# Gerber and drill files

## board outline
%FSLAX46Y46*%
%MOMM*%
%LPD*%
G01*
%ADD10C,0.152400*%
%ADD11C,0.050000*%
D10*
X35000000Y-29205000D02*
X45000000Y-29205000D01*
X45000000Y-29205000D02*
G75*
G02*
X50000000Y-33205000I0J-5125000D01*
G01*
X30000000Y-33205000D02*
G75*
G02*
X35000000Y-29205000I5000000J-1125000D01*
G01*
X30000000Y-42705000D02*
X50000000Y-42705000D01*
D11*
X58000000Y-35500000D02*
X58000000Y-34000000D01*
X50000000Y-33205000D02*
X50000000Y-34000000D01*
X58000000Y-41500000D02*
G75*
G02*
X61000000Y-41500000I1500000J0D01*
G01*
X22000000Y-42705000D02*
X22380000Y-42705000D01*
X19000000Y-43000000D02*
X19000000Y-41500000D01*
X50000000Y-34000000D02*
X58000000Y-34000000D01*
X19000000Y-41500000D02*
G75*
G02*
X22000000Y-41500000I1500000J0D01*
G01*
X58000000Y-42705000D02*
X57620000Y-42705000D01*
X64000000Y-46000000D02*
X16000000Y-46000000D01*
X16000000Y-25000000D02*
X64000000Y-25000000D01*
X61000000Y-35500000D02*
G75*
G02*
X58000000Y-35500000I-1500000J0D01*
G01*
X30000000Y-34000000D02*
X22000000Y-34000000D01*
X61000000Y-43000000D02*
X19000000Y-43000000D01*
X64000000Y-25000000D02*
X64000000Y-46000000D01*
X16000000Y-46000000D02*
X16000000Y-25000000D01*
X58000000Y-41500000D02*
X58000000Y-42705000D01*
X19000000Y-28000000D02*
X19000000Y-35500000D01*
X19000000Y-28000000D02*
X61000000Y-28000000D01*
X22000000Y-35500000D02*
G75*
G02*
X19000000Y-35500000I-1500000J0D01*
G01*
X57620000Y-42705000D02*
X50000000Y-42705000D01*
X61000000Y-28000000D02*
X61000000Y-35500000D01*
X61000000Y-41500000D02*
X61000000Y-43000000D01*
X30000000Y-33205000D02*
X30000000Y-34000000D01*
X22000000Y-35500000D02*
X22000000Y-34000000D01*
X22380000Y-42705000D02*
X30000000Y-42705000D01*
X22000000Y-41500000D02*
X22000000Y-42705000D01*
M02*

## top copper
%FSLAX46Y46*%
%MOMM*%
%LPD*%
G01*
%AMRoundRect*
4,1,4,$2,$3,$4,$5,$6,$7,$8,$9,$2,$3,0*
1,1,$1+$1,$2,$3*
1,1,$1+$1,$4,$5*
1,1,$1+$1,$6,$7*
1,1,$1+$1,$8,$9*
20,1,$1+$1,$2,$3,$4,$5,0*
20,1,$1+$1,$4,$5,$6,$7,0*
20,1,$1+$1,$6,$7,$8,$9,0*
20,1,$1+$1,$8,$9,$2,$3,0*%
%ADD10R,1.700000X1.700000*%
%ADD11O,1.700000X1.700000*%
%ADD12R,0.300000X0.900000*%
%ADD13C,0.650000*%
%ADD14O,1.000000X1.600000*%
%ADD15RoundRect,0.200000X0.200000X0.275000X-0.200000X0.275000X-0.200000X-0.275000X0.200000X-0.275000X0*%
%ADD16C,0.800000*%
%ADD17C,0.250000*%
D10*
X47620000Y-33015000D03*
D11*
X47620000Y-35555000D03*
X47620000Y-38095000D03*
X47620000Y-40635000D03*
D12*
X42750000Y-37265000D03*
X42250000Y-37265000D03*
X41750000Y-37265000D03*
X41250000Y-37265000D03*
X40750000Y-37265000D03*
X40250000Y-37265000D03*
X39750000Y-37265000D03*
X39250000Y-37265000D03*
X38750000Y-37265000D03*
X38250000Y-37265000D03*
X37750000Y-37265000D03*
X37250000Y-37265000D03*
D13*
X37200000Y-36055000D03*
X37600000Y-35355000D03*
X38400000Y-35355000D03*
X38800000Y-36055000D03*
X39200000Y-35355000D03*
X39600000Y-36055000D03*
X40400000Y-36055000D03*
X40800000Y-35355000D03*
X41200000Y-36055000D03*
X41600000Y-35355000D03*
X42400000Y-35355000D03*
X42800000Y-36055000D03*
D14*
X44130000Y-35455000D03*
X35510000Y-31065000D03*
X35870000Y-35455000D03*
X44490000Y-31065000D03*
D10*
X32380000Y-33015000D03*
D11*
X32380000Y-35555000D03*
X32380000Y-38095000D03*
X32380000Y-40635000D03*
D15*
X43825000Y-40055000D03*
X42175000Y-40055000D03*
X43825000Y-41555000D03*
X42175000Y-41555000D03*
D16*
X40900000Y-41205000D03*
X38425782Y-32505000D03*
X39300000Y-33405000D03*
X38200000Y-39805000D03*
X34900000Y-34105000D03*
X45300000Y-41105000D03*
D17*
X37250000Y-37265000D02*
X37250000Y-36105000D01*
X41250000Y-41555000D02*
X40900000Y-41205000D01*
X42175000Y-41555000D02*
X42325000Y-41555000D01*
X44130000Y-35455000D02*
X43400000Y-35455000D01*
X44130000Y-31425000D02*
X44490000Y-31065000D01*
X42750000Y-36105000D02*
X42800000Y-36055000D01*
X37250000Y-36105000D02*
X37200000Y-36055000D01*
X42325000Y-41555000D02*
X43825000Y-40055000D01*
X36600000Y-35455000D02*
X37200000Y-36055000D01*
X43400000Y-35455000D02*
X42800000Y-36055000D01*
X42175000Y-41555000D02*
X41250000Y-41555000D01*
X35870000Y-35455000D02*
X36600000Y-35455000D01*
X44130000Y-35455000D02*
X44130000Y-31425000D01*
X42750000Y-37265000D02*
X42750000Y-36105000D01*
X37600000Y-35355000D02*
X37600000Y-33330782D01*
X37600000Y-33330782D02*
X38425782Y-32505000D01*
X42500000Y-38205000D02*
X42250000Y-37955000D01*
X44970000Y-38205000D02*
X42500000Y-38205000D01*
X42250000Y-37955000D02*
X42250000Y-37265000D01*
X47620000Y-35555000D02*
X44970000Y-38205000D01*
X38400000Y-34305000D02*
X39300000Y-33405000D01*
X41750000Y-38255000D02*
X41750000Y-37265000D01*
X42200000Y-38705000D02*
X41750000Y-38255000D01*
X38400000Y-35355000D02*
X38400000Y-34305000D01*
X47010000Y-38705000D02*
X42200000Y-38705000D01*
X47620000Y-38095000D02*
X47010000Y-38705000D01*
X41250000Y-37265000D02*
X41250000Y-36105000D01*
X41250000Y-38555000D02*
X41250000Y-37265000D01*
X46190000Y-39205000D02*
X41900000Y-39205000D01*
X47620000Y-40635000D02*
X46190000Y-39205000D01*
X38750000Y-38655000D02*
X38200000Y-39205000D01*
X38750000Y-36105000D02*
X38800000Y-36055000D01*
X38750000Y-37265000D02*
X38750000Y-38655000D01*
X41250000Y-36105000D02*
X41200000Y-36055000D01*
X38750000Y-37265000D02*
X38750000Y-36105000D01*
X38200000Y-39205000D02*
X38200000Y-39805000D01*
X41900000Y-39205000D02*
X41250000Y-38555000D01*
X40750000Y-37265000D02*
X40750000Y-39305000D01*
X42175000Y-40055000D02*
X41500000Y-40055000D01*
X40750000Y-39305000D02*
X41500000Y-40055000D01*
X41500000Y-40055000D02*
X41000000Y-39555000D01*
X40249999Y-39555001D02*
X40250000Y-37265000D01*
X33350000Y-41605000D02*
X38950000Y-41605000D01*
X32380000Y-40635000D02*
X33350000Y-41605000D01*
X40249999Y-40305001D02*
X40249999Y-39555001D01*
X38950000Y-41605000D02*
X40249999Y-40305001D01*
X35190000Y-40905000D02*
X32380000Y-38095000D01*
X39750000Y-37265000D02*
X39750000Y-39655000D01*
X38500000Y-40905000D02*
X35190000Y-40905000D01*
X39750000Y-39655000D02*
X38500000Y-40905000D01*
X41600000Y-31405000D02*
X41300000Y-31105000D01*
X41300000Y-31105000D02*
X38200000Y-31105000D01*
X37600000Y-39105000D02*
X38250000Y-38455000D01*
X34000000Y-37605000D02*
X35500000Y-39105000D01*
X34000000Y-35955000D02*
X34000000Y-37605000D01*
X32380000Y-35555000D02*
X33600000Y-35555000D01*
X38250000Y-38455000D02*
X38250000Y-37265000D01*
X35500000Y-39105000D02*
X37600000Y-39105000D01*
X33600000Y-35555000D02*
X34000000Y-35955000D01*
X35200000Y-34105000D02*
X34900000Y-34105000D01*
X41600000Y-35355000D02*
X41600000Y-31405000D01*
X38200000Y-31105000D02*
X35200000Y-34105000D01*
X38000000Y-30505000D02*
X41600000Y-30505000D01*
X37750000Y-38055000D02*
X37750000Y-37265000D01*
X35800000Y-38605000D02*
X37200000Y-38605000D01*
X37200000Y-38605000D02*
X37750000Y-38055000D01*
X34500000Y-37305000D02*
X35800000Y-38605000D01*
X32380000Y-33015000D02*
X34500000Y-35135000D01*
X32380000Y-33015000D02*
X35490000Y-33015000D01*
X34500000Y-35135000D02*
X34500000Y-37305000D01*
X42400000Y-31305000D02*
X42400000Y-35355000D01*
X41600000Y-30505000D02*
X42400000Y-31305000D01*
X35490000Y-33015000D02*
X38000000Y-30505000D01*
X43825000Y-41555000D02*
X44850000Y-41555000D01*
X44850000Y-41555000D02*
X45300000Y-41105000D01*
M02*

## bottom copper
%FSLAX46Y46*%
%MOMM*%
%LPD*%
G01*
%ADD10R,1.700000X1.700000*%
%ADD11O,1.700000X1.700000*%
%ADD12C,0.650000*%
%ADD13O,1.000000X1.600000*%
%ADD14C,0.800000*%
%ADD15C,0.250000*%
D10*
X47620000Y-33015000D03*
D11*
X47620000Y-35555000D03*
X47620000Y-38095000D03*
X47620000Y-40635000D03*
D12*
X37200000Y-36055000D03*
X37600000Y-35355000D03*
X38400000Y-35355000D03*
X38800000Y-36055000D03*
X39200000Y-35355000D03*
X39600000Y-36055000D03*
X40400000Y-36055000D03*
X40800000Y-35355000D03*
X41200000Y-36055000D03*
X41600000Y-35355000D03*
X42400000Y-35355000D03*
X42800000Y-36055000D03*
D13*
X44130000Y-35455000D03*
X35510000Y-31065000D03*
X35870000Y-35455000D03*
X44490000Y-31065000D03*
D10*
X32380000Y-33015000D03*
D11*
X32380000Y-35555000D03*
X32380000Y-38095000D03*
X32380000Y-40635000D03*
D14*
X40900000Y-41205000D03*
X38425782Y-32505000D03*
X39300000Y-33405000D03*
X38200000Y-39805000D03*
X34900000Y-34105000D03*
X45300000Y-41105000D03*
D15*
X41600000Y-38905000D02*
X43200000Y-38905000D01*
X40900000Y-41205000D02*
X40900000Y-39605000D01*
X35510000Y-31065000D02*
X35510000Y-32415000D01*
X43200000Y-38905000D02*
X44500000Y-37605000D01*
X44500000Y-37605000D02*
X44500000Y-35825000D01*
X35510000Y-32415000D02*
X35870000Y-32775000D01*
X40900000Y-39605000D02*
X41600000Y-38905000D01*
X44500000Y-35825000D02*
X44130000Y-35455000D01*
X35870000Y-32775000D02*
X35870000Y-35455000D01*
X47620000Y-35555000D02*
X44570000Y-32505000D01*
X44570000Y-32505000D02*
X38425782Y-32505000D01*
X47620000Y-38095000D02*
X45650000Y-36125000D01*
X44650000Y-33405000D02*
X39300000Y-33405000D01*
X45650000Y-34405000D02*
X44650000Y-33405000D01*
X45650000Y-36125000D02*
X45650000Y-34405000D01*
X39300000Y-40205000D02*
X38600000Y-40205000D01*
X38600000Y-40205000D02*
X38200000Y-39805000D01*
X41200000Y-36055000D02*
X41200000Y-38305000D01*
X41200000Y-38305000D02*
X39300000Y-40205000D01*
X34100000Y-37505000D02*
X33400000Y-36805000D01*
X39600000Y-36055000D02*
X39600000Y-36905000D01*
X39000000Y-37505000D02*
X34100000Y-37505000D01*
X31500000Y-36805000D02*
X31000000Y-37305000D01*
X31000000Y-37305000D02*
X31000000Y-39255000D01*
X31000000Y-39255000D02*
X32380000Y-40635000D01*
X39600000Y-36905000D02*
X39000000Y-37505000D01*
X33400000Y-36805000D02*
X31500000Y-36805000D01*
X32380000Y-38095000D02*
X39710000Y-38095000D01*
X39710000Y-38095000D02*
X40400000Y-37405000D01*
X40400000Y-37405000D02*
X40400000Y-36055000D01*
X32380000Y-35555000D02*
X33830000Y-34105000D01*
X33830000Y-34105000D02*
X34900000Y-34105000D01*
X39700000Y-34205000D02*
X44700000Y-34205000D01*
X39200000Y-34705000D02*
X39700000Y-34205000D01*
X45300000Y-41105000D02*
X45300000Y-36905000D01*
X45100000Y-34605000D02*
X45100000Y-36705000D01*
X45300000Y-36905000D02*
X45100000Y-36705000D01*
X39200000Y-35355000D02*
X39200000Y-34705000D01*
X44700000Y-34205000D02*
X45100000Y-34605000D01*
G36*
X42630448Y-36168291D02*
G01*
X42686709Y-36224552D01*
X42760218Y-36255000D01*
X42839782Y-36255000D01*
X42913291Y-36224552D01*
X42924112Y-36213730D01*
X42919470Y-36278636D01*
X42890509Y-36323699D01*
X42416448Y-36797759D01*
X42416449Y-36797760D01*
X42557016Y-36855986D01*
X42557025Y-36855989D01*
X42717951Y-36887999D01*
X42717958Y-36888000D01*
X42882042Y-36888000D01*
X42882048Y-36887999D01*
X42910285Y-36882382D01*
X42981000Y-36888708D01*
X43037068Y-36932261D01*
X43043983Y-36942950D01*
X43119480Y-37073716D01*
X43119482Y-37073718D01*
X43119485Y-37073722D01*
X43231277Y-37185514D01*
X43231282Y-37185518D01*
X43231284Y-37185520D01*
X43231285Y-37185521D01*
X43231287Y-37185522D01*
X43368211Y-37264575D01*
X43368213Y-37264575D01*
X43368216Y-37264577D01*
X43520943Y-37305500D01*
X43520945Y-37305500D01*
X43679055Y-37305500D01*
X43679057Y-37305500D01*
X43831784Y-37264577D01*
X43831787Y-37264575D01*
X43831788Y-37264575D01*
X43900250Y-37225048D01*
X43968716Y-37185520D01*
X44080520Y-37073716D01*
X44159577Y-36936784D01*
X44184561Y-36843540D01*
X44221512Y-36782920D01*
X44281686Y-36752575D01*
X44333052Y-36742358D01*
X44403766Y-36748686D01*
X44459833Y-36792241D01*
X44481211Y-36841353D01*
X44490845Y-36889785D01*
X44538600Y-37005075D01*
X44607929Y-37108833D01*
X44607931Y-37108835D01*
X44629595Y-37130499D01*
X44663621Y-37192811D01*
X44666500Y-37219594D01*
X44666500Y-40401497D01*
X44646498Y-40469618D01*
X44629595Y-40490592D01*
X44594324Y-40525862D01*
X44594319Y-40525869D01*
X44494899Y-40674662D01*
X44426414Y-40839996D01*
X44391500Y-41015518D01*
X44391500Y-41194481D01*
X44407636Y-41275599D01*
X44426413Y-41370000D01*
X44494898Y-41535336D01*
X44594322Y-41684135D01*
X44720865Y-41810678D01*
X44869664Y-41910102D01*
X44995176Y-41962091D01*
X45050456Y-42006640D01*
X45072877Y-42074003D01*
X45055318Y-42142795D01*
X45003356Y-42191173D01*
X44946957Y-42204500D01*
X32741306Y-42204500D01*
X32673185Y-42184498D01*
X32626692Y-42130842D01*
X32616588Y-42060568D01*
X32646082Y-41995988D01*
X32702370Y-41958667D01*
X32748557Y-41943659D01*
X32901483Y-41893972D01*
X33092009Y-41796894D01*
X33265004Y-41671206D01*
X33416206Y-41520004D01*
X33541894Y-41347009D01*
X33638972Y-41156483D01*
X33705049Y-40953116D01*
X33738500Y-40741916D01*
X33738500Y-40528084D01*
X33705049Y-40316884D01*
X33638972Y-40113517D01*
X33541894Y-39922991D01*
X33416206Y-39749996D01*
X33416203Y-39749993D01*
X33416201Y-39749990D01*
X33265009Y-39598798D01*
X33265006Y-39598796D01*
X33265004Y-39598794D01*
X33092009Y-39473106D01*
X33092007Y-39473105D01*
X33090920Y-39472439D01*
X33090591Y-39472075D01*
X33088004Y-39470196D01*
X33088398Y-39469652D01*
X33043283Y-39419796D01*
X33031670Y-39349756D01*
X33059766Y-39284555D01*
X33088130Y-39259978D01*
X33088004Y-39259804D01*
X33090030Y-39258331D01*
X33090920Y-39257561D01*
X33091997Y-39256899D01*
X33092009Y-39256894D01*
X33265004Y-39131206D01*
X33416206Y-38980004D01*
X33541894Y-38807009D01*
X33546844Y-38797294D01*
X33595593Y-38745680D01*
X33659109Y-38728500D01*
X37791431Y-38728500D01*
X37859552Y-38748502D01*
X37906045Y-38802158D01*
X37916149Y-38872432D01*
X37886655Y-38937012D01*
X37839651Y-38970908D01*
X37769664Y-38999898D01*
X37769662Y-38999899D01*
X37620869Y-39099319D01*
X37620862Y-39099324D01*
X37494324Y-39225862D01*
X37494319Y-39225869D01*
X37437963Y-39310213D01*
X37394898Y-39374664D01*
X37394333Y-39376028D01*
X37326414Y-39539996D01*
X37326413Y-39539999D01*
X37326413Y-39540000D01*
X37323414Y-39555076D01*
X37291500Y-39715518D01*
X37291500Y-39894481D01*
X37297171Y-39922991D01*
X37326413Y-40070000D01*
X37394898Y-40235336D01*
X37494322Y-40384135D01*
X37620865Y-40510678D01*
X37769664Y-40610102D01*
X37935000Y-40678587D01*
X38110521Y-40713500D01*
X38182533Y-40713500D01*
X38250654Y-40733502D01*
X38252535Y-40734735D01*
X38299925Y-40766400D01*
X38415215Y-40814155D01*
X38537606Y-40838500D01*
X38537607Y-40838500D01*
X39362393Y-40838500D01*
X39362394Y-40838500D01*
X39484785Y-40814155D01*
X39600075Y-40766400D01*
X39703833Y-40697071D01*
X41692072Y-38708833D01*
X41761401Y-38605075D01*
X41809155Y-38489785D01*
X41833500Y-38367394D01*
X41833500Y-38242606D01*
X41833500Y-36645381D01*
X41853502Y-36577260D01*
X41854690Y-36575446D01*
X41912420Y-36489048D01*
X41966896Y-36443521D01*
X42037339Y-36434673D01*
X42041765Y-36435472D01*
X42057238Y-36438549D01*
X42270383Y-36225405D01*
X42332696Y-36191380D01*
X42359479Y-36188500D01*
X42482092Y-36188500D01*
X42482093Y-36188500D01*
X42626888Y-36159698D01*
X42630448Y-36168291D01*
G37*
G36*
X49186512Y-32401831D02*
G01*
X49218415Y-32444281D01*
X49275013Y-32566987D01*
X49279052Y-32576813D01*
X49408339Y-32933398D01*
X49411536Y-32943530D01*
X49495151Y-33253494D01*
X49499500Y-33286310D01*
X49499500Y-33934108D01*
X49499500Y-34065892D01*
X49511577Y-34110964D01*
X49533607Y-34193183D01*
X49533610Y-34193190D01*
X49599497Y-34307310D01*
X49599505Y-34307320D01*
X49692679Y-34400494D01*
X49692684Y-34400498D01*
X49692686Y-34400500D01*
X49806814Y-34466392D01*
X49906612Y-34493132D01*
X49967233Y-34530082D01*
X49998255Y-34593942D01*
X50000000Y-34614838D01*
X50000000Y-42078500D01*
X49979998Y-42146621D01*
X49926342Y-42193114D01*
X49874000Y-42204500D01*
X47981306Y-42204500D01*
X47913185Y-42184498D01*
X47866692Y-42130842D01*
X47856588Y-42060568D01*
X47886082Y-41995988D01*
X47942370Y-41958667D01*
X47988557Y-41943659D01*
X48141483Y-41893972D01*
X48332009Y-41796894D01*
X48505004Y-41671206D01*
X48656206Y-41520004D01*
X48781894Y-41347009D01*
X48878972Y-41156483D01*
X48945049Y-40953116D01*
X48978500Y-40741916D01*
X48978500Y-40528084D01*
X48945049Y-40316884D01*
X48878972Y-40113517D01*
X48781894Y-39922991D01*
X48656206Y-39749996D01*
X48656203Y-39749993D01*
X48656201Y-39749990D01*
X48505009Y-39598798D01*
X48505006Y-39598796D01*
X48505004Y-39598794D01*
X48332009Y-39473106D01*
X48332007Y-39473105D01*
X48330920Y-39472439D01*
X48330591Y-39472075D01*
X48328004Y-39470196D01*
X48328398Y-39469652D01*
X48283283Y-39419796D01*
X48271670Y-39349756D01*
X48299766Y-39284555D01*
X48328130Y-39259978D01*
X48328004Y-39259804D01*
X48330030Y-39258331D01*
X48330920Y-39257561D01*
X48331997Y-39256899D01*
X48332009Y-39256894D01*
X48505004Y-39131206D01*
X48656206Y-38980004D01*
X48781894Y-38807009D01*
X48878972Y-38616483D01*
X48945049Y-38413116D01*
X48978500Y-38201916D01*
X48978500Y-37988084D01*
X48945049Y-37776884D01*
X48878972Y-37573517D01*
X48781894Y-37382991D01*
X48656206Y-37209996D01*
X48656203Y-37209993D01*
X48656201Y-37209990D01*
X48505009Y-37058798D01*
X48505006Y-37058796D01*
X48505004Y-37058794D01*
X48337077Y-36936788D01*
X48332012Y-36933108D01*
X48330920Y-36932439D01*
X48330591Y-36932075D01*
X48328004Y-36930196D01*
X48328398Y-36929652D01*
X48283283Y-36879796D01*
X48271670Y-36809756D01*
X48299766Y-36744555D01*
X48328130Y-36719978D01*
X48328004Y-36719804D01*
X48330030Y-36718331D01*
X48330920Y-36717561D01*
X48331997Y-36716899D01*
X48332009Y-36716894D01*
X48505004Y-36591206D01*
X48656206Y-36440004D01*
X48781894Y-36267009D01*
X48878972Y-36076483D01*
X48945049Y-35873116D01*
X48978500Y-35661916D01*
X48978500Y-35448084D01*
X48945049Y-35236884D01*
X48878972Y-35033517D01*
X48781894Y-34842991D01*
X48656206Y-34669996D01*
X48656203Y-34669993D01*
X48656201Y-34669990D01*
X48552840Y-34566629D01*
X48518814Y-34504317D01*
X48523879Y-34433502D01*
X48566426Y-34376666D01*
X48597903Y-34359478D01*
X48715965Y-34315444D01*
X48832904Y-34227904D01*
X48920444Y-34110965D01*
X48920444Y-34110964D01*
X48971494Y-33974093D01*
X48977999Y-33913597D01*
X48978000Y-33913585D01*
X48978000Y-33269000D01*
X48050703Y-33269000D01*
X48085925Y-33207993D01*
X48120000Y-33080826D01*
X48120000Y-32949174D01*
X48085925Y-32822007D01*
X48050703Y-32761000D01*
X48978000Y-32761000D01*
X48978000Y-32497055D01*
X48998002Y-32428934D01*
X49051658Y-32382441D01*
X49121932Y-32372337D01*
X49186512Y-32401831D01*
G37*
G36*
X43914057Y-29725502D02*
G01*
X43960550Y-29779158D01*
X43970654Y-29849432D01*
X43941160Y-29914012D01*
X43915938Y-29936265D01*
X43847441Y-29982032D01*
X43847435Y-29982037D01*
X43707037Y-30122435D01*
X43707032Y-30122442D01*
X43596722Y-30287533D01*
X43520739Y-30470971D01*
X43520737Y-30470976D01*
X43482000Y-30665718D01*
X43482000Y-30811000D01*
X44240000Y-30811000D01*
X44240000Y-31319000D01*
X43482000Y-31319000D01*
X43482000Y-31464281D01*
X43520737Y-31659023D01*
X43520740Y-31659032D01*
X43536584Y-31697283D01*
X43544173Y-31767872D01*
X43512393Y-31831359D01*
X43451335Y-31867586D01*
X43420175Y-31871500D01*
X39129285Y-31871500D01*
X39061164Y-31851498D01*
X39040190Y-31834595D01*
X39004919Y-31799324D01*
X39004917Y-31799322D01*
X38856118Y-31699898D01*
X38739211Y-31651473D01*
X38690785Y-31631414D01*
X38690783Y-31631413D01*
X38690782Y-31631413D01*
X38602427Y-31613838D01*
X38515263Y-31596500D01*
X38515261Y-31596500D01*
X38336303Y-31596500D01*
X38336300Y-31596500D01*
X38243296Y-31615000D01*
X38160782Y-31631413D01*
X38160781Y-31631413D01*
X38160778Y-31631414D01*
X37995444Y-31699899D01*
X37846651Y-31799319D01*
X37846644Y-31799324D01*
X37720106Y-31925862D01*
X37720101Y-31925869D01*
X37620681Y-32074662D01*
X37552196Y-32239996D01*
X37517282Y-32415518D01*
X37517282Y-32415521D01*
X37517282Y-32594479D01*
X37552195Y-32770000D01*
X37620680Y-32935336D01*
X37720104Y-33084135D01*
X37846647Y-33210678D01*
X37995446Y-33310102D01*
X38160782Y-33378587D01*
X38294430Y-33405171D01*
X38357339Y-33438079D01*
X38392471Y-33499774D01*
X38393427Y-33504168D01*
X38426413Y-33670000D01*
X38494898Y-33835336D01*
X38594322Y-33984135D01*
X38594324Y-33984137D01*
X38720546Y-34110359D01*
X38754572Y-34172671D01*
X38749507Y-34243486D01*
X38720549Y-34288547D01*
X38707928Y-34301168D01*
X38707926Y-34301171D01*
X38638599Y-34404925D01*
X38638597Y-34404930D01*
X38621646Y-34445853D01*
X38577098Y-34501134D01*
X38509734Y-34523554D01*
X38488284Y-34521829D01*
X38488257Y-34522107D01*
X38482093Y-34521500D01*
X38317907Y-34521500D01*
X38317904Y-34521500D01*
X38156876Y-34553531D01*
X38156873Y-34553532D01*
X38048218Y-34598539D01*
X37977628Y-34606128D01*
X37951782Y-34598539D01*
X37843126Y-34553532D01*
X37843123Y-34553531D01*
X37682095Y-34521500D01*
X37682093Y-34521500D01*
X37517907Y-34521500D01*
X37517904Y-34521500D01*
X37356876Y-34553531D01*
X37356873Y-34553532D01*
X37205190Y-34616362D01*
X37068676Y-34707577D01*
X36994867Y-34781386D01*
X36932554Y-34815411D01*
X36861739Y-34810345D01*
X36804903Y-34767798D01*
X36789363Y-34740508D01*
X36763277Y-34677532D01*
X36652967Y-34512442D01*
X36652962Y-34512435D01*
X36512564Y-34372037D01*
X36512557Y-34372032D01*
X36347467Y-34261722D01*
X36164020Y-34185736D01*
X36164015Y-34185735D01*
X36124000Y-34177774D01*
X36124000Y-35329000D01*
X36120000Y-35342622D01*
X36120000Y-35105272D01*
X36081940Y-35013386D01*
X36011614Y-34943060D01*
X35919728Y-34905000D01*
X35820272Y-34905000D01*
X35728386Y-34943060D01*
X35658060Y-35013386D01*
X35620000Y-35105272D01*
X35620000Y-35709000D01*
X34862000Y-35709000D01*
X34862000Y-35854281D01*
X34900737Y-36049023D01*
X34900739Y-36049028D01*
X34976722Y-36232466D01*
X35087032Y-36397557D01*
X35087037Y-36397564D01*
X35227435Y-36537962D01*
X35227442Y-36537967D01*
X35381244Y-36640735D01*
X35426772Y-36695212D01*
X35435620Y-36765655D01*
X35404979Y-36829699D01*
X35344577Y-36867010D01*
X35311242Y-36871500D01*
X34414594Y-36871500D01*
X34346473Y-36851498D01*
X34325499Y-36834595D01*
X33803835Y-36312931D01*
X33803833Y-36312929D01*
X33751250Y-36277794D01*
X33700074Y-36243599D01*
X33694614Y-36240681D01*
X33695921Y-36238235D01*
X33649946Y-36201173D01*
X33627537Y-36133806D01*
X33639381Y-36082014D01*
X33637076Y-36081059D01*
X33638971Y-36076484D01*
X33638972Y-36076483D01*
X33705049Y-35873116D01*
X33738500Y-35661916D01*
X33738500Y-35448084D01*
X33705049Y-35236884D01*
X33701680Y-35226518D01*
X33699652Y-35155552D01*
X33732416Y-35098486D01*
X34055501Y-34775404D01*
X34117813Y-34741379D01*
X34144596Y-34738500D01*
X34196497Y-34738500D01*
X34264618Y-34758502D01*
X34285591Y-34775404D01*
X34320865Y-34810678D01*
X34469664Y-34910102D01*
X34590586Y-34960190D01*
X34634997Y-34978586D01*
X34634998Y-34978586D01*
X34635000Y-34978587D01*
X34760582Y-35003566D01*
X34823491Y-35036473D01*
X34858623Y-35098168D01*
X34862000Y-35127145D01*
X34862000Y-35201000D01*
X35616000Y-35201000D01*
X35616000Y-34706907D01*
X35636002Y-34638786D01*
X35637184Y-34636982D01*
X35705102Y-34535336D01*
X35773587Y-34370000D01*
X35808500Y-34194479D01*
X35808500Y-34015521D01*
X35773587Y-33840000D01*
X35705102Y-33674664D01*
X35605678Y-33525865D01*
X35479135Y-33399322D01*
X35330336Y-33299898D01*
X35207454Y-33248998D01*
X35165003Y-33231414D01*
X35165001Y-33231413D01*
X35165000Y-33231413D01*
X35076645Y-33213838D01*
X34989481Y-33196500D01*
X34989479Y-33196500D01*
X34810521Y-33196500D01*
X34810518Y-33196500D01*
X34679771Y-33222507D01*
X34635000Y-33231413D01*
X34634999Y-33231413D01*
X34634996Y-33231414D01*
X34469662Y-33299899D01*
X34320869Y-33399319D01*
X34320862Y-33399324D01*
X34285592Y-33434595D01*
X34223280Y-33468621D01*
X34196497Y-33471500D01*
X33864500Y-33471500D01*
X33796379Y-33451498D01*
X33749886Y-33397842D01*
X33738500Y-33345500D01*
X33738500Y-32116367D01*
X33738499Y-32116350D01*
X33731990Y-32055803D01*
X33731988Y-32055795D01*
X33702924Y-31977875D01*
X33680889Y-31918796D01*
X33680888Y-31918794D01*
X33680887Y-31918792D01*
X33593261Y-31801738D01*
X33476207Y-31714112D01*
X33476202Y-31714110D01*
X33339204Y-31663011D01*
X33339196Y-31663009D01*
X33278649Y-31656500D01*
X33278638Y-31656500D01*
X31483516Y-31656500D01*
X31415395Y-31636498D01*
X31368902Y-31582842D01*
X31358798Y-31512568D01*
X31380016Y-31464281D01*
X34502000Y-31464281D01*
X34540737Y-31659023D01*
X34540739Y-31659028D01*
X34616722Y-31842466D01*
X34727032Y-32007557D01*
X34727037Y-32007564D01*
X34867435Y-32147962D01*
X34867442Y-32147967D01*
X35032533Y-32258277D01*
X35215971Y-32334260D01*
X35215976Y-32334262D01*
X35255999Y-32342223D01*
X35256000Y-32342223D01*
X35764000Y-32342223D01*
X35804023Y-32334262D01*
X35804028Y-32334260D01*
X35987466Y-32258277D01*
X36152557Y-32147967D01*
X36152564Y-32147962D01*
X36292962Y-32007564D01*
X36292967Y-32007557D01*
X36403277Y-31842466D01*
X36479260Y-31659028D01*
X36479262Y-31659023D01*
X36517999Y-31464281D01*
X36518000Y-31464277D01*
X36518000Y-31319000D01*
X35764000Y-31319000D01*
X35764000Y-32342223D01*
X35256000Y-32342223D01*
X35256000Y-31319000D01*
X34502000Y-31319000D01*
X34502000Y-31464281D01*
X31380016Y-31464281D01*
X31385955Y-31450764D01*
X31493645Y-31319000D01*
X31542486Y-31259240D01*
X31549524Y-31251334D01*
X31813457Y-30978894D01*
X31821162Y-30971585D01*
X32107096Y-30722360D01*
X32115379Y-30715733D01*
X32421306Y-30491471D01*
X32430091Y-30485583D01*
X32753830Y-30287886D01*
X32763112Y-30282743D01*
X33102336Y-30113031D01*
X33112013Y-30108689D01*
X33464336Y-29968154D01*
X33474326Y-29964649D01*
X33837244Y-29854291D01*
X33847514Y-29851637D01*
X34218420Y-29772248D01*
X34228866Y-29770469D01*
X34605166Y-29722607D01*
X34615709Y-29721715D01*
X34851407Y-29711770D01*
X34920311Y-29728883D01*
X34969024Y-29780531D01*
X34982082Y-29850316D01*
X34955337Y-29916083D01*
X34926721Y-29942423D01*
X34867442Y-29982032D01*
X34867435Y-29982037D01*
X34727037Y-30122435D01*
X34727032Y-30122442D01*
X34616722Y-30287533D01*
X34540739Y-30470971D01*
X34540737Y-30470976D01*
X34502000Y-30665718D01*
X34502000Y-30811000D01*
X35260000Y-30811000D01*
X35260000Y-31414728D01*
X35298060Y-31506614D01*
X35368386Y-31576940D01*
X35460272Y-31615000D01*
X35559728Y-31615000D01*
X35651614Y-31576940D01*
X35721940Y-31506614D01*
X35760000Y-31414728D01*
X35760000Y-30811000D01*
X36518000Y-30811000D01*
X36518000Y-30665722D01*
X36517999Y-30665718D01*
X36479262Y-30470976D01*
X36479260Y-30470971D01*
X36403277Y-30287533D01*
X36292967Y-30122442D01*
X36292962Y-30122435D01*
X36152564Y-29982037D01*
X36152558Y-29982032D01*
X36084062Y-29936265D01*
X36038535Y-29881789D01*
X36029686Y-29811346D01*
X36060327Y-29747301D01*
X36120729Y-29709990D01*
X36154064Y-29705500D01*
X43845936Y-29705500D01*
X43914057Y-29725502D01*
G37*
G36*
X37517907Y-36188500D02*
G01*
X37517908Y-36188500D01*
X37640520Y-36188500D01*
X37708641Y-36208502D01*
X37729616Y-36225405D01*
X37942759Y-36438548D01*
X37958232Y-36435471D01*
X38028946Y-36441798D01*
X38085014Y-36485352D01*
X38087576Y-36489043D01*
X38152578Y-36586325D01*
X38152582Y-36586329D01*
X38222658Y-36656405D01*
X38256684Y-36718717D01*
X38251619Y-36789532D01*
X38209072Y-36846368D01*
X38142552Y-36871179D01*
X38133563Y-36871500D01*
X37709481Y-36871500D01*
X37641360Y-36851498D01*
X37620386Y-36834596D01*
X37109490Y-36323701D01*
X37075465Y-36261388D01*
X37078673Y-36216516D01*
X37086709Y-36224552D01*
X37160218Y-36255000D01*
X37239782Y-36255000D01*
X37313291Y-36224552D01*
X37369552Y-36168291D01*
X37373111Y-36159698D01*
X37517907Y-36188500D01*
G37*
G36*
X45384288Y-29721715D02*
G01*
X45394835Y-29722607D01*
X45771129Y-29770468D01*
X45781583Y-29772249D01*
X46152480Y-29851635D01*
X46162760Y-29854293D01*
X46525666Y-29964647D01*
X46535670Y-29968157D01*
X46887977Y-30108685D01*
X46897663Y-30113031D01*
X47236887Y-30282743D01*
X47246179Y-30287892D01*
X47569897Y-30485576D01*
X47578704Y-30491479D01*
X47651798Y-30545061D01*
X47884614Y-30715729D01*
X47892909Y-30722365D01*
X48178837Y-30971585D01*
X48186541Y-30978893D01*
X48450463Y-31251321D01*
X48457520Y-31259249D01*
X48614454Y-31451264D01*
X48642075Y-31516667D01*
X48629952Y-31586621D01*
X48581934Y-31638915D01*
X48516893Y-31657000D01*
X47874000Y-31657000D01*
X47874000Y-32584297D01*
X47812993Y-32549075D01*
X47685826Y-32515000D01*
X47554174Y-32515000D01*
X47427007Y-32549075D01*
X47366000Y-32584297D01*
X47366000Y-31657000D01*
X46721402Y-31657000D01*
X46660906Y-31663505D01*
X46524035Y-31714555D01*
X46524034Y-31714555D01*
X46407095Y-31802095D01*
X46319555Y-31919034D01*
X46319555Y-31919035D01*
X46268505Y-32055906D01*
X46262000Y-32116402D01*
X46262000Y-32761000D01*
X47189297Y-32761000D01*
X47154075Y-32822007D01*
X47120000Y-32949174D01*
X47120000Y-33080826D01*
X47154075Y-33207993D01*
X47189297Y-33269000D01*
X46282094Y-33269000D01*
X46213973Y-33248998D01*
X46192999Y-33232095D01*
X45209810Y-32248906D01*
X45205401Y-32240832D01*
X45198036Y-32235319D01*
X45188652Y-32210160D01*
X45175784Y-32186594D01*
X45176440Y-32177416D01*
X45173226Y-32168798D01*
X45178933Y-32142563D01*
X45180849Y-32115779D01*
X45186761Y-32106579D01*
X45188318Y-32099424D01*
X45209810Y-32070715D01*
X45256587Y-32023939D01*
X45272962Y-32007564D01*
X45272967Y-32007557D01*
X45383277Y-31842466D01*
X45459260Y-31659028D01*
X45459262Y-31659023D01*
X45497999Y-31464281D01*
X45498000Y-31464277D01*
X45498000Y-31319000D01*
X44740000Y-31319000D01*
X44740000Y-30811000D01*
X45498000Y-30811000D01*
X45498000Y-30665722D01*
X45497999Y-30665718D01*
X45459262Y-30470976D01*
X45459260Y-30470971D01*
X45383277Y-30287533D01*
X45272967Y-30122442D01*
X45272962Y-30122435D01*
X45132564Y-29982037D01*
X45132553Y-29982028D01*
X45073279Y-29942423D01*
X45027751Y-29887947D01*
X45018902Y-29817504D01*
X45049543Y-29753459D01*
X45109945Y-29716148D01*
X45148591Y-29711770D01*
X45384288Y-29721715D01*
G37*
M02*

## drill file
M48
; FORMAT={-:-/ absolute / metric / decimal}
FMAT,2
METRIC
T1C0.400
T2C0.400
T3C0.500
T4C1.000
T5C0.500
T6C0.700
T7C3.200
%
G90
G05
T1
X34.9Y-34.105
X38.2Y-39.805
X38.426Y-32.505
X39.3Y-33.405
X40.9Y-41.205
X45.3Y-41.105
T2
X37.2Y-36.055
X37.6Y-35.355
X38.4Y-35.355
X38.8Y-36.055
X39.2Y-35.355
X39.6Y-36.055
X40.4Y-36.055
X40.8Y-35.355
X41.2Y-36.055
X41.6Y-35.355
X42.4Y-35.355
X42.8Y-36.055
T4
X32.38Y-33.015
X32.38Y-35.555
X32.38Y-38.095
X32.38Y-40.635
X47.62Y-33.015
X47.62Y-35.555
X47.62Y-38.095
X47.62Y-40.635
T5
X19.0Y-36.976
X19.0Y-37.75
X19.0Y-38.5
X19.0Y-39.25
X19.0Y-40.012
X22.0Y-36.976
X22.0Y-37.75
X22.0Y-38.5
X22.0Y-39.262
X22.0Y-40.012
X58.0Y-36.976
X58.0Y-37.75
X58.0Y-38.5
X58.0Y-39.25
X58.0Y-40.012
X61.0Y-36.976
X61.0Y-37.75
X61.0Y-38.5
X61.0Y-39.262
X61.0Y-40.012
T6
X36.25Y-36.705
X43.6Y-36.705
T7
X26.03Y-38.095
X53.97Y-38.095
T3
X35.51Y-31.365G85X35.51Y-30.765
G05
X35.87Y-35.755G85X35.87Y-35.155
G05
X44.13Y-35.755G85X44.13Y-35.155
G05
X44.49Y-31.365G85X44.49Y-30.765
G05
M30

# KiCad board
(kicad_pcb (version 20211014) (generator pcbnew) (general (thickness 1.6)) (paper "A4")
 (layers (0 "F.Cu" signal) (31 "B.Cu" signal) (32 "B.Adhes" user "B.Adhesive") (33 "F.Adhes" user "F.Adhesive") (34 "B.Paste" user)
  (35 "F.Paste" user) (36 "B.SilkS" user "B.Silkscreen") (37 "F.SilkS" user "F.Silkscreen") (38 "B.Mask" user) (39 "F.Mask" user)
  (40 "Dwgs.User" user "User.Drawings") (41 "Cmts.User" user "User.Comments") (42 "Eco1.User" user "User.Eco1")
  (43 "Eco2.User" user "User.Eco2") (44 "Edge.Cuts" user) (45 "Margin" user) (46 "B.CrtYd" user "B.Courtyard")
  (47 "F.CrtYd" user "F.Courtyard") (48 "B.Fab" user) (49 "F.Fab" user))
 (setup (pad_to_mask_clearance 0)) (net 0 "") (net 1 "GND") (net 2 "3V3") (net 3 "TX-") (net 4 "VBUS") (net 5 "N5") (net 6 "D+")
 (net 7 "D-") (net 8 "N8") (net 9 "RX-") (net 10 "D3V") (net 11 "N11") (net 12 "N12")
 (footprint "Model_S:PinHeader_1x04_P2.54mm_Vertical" (layer "F.Cu") (at 47.62 33.015)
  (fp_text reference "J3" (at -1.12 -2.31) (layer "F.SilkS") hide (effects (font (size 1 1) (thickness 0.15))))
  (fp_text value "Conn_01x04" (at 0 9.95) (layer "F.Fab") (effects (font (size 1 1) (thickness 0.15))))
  (pad "1" thru_hole rect locked (at 0 0) (size 1.7 1.7) (drill 1) (layers *.Cu *.Mask) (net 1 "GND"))
  (pad "2" thru_hole oval locked (at 0 2.54) (size 1.7 1.7) (drill 1) (layers *.Cu *.Mask) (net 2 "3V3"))
  (pad "3" thru_hole oval locked (at 0 5.08) (size 1.7 1.7) (drill 1) (layers *.Cu *.Mask) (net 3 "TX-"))
  (pad "4" thru_hole oval locked (at 0 7.62) (size 1.7 1.7) (drill 1) (layers *.Cu *.Mask) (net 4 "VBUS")))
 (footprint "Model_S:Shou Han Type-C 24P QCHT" (layer "F.Cu") (at 40 29.205 180)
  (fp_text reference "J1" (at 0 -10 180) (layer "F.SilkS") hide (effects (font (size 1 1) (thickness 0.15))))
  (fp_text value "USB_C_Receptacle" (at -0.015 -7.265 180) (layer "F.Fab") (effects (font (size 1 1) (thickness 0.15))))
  (pad "" np_thru_hole circle locked (at -3.6 -7.5 180) (size 0.7 0.7) (drill 0.7) (layers *.Cu *.Mask))
  (pad "" np_thru_hole circle locked (at 3.75 -7.5 180) (size 0.7 0.7) (drill 0.7) (layers *.Cu *.Mask))
  (pad "A1" smd rect locked (at -2.75 -8.06 180) (size 0.3 0.9) (layers "F.Cu" "F.Paste" "F.Mask") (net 1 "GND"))
  (pad "A2" smd rect locked (at -2.25 -8.06 180) (size 0.3 0.9) (layers "F.Cu" "F.Paste" "F.Mask") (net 2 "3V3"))
  (pad "A3" smd rect locked (at -1.75 -8.06 180) (size 0.3 0.9) (layers "F.Cu" "F.Paste" "F.Mask") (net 3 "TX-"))
  (pad "A4" smd rect locked (at -1.25 -8.06 180) (size 0.3 0.9) (layers "F.Cu" "F.Paste" "F.Mask") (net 4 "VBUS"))
  (pad "A5" smd rect locked (at -0.75 -8.06 180) (size 0.3 0.9) (layers "F.Cu" "F.Paste" "F.Mask") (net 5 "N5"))
  (pad "A6" smd rect locked (at -0.25 -8.06 180) (size 0.3 0.9) (layers "F.Cu" "F.Paste" "F.Mask") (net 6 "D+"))
  (pad "A7" smd rect locked (at 0.25 -8.06 180) (size 0.3 0.9) (layers "F.Cu" "F.Paste" "F.Mask") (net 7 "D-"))
  (pad "A8" smd rect locked (at 0.75 -8.06 180) (size 0.3 0.9) (layers "F.Cu" "F.Paste" "F.Mask") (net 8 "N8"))
  (pad "A9" smd rect locked (at 1.25 -8.06 180) (size 0.3 0.9) (layers "F.Cu" "F.Paste" "F.Mask") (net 4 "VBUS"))
  (pad "A10" smd rect locked (at 1.75 -8.06 180) (size 0.3 0.9) (layers "F.Cu" "F.Paste" "F.Mask") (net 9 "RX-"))
  (pad "A11" smd rect locked (at 2.25 -8.06 180) (size 0.3 0.9) (layers "F.Cu" "F.Paste" "F.Mask") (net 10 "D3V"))
  (pad "A12" smd rect locked (at 2.75 -8.06 180) (size 0.3 0.9) (layers "F.Cu" "F.Paste" "F.Mask") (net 1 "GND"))
  (pad "B1" thru_hole circle locked (at 2.8 -6.85 180) (size 0.65 0.65) (drill 0.4) (layers *.Cu *.Mask) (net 1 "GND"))
  (pad "B2" thru_hole circle locked (at 2.4 -6.15 180) (size 0.65 0.65) (drill 0.4) (layers *.Cu *.Mask) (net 2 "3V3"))
  (pad "B3" thru_hole circle locked (at 1.6 -6.15 180) (size 0.65 0.65) (drill 0.4) (layers *.Cu *.Mask) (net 3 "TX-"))
  (pad "B4" thru_hole circle locked (at 1.2 -6.85 180) (size 0.65 0.65) (drill 0.4) (layers *.Cu *.Mask) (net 4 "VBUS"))
  (pad "B5" thru_hole circle locked (at 0.8 -6.15 180) (size 0.65 0.65) (drill 0.4) (layers *.Cu *.Mask) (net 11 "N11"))
  (pad "B6" thru_hole circle locked (at 0.4 -6.85 180) (size 0.65 0.65) (drill 0.4) (layers *.Cu *.Mask) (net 6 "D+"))
  (pad "B7" thru_hole circle locked (at -0.4 -6.85 180) (size 0.65 0.65) (drill 0.4) (layers *.Cu *.Mask) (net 7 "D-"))
  (pad "B8" thru_hole circle locked (at -0.8 -6.15 180) (size 0.65 0.65) (drill 0.4) (layers *.Cu *.Mask) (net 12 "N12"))
  (pad "B9" thru_hole circle locked (at -1.2 -6.85 180) (size 0.65 0.65) (drill 0.4) (layers *.Cu *.Mask) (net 4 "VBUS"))
  (pad "B10" thru_hole circle locked (at -1.6 -6.15 180) (size 0.65 0.65) (drill 0.4) (layers *.Cu *.Mask) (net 9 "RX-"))
  (pad "B11" thru_hole circle locked (at -2.4 -6.15 180) (size 0.65 0.65) (drill 0.4) (layers *.Cu *.Mask) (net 10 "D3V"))
  (pad "B12" thru_hole circle locked (at -2.8 -6.85 180) (size 0.65 0.65) (drill 0.4) (layers *.Cu *.Mask) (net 1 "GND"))
  (pad "S1" thru_hole oval locked (at -4.13 -6.25 180) (size 1 1.6) (drill oval 0.5 1.1) (layers *.Cu *.Mask) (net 1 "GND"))
  (pad "S1" thru_hole oval locked (at 4.49 -1.86 180) (size 1 1.6) (drill oval 0.5 1.1) (layers *.Cu *.Mask) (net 1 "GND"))
  (pad "S1" thru_hole oval locked (at 4.13 -6.25 180) (size 1 1.6) (drill oval 0.5 1.1) (layers *.Cu *.Mask) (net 1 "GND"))
  (pad "S1" thru_hole oval locked (at -4.49 -1.86 180) (size 1 1.6) (drill oval 0.5 1.1) (layers *.Cu *.Mask) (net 1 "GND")))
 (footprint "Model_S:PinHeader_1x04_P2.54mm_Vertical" (layer "F.Cu") (at 32.38 33.015)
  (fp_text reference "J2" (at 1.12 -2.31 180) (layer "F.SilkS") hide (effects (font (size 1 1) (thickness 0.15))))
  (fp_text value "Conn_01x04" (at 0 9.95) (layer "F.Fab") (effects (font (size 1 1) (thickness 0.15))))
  (pad "1" thru_hole rect locked (at 0 0) (size 1.7 1.7) (drill 1) (layers *.Cu *.Mask) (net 10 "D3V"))
  (pad "2" thru_hole oval locked (at 0 2.54) (size 1.7 1.7) (drill 1) (layers *.Cu *.Mask) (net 9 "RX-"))
  (pad "3" thru_hole oval locked (at 0 5.08) (size 1.7 1.7) (drill 1) (layers *.Cu *.Mask) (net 7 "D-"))
  (pad "4" thru_hole oval locked (at 0 7.62) (size 1.7 1.7) (drill 1) (layers *.Cu *.Mask) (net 6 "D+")))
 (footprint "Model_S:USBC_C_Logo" (layer "F.Cu") (at 40 40)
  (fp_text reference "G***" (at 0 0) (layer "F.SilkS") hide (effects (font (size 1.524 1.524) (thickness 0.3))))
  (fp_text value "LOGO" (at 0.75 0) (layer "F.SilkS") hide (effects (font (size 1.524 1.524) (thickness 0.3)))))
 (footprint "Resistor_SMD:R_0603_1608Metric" (layer "F.Cu") (at 43 40.055 180)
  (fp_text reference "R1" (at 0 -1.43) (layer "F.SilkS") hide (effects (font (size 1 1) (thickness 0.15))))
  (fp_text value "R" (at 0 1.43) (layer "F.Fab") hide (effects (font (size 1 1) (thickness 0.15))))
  (pad "1" smd roundrect locked (at -0.825 0 180) (size 0.8 0.95) (layers "F.Cu" "F.Paste" "F.Mask") (roundrect_rratio 0.25) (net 1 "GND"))
  (pad "2" smd roundrect locked (at 0.825 0 180) (size 0.8 0.95) (layers "F.Cu" "F.Paste" "F.Mask") (roundrect_rratio 0.25) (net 5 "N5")))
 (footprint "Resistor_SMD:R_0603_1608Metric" (layer "F.Cu") (at 43 41.555 180)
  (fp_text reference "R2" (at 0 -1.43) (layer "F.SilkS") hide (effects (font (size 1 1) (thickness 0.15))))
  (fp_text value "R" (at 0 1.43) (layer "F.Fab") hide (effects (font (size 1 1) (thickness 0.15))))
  (pad "1" smd roundrect locked (at -0.825 0 180) (size 0.8 0.95) (layers "F.Cu" "F.Paste" "F.Mask") (roundrect_rratio 0.25) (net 11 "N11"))
  (pad "2" smd roundrect locked (at 0.825 0 180) (size 0.8 0.95) (layers "F.Cu" "F.Paste" "F.Mask") (roundrect_rratio 0.25) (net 1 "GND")))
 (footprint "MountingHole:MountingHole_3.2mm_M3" (layer "F.Cu") (at 26.03 38.095)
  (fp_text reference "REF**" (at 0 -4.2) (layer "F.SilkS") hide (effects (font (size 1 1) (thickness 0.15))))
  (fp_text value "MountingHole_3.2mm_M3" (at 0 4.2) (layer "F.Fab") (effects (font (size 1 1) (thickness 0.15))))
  (pad "" np_thru_hole circle (at 0 0) (size 3.2 3.2) (drill 3.2) (layers *.Cu *.Mask)))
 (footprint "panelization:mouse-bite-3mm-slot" (layer "F.Cu") (at 20.5 38.5 90)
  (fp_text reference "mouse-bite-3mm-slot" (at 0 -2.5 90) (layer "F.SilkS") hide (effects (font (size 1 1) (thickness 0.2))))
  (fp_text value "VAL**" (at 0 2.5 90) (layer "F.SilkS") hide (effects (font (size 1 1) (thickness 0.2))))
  (pad "" np_thru_hole circle locked (at -1.512 -1.5 90) (size 0.5 0.5) (drill 0.5) (layers *.Cu *.Mask))
  (pad "" np_thru_hole circle locked (at 0 -1.5 90) (size 0.5 0.5) (drill 0.5) (layers *.Cu *.Mask))
  (pad "" np_thru_hole circle locked (at 0.75 1.5 90) (size 0.5 0.5) (drill 0.5) (layers *.Cu *.Mask))
  (pad "" np_thru_hole circle locked (at -1.512 1.5 90) (size 0.5 0.5) (drill 0.5) (layers *.Cu *.Mask))
  (pad "" np_thru_hole circle locked (at 0 1.5 90) (size 0.5 0.5) (drill 0.5) (layers *.Cu *.Mask))
  (pad "" np_thru_hole circle locked (at -0.75 -1.5 90) (size 0.5 0.5) (drill 0.5) (layers *.Cu *.Mask))
  (pad "" np_thru_hole circle locked (at -0.762 1.5 90) (size 0.5 0.5) (drill 0.5) (layers *.Cu *.Mask))
  (pad "" np_thru_hole circle locked (at 1.524 -1.5 90) (size 0.5 0.5) (drill 0.5) (layers *.Cu *.Mask))
  (pad "" np_thru_hole circle locked (at 1.524 1.5 90) (size 0.5 0.5) (drill 0.5) (layers *.Cu *.Mask))
  (pad "" np_thru_hole circle locked (at 0.75 -1.5 90) (size 0.5 0.5) (drill 0.5) (layers *.Cu *.Mask)))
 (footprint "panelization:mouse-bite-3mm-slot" (layer "F.Cu") (at 59.5 38.5 90)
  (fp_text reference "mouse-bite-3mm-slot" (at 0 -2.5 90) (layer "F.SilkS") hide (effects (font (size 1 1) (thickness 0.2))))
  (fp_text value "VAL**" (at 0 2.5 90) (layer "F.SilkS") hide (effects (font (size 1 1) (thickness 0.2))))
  (pad "" np_thru_hole circle locked (at 0 -1.5 90) (size 0.5 0.5) (drill 0.5) (layers *.Cu *.Mask))
  (pad "" np_thru_hole circle locked (at -1.512 1.5 90) (size 0.5 0.5) (drill 0.5) (layers *.Cu *.Mask))
  (pad "" np_thru_hole circle locked (at 0.75 -1.5 90) (size 0.5 0.5) (drill 0.5) (layers *.Cu *.Mask))
  (pad "" np_thru_hole circle locked (at -1.512 -1.5 90) (size 0.5 0.5) (drill 0.5) (layers *.Cu *.Mask))
  (pad "" np_thru_hole circle locked (at 0.75 1.5 90) (size 0.5 0.5) (drill 0.5) (layers *.Cu *.Mask))
  (pad "" np_thru_hole circle locked (at -0.75 -1.5 90) (size 0.5 0.5) (drill 0.5) (layers *.Cu *.Mask))
  (pad "" np_thru_hole circle locked (at 1.524 1.5 90) (size 0.5 0.5) (drill 0.5) (layers *.Cu *.Mask))
  (pad "" np_thru_hole circle locked (at 0 1.5 90) (size 0.5 0.5) (drill 0.5) (layers *.Cu *.Mask))
  (pad "" np_thru_hole circle locked (at -0.762 1.5 90) (size 0.5 0.5) (drill 0.5) (layers *.Cu *.Mask))
  (pad "" np_thru_hole circle locked (at 1.524 -1.5 90) (size 0.5 0.5) (drill 0.5) (layers *.Cu *.Mask)))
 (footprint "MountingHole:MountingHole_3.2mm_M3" (layer "F.Cu") (at 53.97 38.095)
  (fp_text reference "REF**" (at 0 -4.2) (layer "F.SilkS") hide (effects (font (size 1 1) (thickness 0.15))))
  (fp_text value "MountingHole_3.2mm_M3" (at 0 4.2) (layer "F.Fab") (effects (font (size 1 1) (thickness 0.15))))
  (pad "" np_thru_hole circle (at 0 0) (size 3.2 3.2) (drill 3.2) (layers *.Cu *.Mask)))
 (gr_line (start 35 29.205) (end 45 29.205) (layer "Edge.Cuts") (width 0.1524))
 (gr_arc (start 45 29.205) (mid 48.201562 30.328047) (end 50 33.205) (layer "Edge.Cuts") (width 0.1524))
 (gr_arc (start 30 33.205) (mid 31.798438 30.328047) (end 35 29.205) (layer "Edge.Cuts") (width 0.1524))
 (gr_line (start 30 42.705) (end 50 42.705) (layer "Edge.Cuts") (width 0.1524))
 (gr_line (start 58 35.5) (end 58 34) (layer "Edge.Cuts") (width 0.05))
 (gr_line (start 50 33.205) (end 50 34) (layer "Edge.Cuts") (width 0.05))
 (gr_arc (start 58 41.5) (mid 59.5 40) (end 61 41.5) (layer "Edge.Cuts") (width 0.05))
 (gr_line (start 22 42.705) (end 22.38 42.705) (layer "Edge.Cuts") (width 0.05))
 (gr_line (start 19 43) (end 19 41.5) (layer "Edge.Cuts") (width 0.05))
 (gr_line (start 50 34) (end 58 34) (layer "Edge.Cuts") (width 0.05))
 (gr_arc (start 19 41.5) (mid 20.5 40) (end 22 41.5) (layer "Edge.Cuts") (width 0.05))
 (gr_line (start 58 42.705) (end 57.62 42.705) (layer "Edge.Cuts") (width 0.05))
 (gr_line (start 64 46) (end 16 46) (layer "Edge.Cuts") (width 0.05))
 (gr_line (start 16 25) (end 64 25) (layer "Edge.Cuts") (width 0.05))
 (gr_arc (start 61 35.5) (mid 59.5 37) (end 58 35.5) (layer "Edge.Cuts") (width 0.05))
 (gr_line (start 30 34) (end 22 34) (layer "Edge.Cuts") (width 0.05))
 (gr_line (start 61 43) (end 19 43) (layer "Edge.Cuts") (width 0.05))
 (gr_line (start 64 25) (end 64 46) (layer "Edge.Cuts") (width 0.05))
 (gr_line (start 16 46) (end 16 25) (layer "Edge.Cuts") (width 0.05))
 (gr_line (start 58 41.5) (end 58 42.705) (layer "Edge.Cuts") (width 0.05))
 (gr_line (start 19 28) (end 19 35.5) (layer "Edge.Cuts") (width 0.05))
 (gr_line (start 19 28) (end 61 28) (layer "Edge.Cuts") (width 0.05))
 (gr_arc (start 22 35.5) (mid 20.5 37) (end 19 35.5) (layer "Edge.Cuts") (width 0.05))
 (gr_line (start 57.62 42.705) (end 50 42.705) (layer "Edge.Cuts") (width 0.05))
 (gr_line (start 61 28) (end 61 35.5) (layer "Edge.Cuts") (width 0.05))
 (gr_line (start 61 41.5) (end 61 43) (layer "Edge.Cuts") (width 0.05))
 (gr_line (start 30 33.205) (end 30 34) (layer "Edge.Cuts") (width 0.05))
 (gr_line (start 22 35.5) (end 22 34) (layer "Edge.Cuts") (width 0.05))
 (gr_line (start 22.38 42.705) (end 30 42.705) (layer "Edge.Cuts") (width 0.05))
 (gr_line (start 22 41.5) (end 22 42.705) (layer "Edge.Cuts") (width 0.05))
 (segment (start 37.25 37.265) (end 37.25 36.105) (width 0.25) (layer "F.Cu") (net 1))
 (segment (start 41.25 41.555) (end 40.9 41.205) (width 0.25) (layer "F.Cu") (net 1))
 (segment (start 42.175 41.555) (end 42.325 41.555) (width 0.25) (layer "F.Cu") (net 1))
 (segment (start 44.13 35.455) (end 43.4 35.455) (width 0.25) (layer "F.Cu") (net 1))
 (segment (start 44.13 31.425) (end 44.49 31.065) (width 0.25) (layer "F.Cu") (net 1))
 (segment (start 42.75 36.105) (end 42.8 36.055) (width 0.25) (layer "F.Cu") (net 1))
 (segment (start 37.25 36.105) (end 37.2 36.055) (width 0.25) (layer "F.Cu") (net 1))
 (segment (start 42.325 41.555) (end 43.825 40.055) (width 0.25) (layer "F.Cu") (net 1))
 (segment (start 36.6 35.455) (end 37.2 36.055) (width 0.25) (layer "F.Cu") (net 1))
 (segment (start 43.4 35.455) (end 42.8 36.055) (width 0.25) (layer "F.Cu") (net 1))
 (segment (start 42.175 41.555) (end 41.25 41.555) (width 0.25) (layer "F.Cu") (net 1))
 (segment (start 35.87 35.455) (end 36.6 35.455) (width 0.25) (layer "F.Cu") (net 1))
 (segment (start 44.13 35.455) (end 44.13 31.425) (width 0.25) (layer "F.Cu") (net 1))
 (segment (start 42.75 37.265) (end 42.75 36.105) (width 0.25) (layer "F.Cu") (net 1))
 (via (at 40.9 41.205) (size 0.8) (drill 0.4) (layers "F.Cu" "B.Cu") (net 1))
 (segment (start 41.6 38.905) (end 43.2 38.905) (width 0.25) (layer "B.Cu") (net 1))
 (segment (start 40.9 41.205) (end 40.9 39.605) (width 0.25) (layer "B.Cu") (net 1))
 (segment (start 35.51 31.065) (end 35.51 32.415) (width 0.25) (layer "B.Cu") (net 1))
 (segment (start 43.2 38.905) (end 44.5 37.605) (width 0.25) (layer "B.Cu") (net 1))
 (segment (start 44.5 37.605) (end 44.5 35.825) (width 0.25) (layer "B.Cu") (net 1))
 (segment (start 35.51 32.415) (end 35.87 32.775) (width 0.25) (layer "B.Cu") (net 1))
 (segment (start 40.9 39.605) (end 41.6 38.905) (width 0.25) (layer "B.Cu") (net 1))
 (segment (start 44.5 35.825) (end 44.13 35.455) (width 0.25) (layer "B.Cu") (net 1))
 (segment (start 35.87 32.775) (end 35.87 35.455) (width 0.25) (layer "B.Cu") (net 1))
 (segment (start 37.6 35.355) (end 37.6 33.330782) (width 0.25) (layer "F.Cu") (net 2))
 (segment (start 37.6 33.330782) (end 38.425782 32.505) (width 0.25) (layer "F.Cu") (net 2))
 (segment (start 42.5 38.205) (end 42.25 37.955) (width 0.25) (layer "F.Cu") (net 2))
 (segment (start 44.97 38.205) (end 42.5 38.205) (width 0.25) (layer "F.Cu") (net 2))
 (segment (start 42.25 37.955) (end 42.25 37.265) (width 0.25) (layer "F.Cu") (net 2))
 (segment (start 47.62 35.555) (end 44.97 38.205) (width 0.25) (layer "F.Cu") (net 2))
 (via (at 38.425782 32.505) (size 0.8) (drill 0.4) (layers "F.Cu" "B.Cu") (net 2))
 (segment (start 47.62 35.555) (end 44.57 32.505) (width 0.25) (layer "B.Cu") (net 2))
 (segment (start 44.57 32.505) (end 38.425782 32.505) (width 0.25) (layer "B.Cu") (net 2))
 (segment (start 38.4 34.305) (end 39.3 33.405) (width 0.25) (layer "F.Cu") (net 3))
 (segment (start 41.75 38.255) (end 41.75 37.265) (width 0.25) (layer "F.Cu") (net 3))
 (segment (start 42.2 38.705) (end 41.75 38.255) (width 0.25) (layer "F.Cu") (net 3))
 (segment (start 38.4 35.355) (end 38.4 34.305) (width 0.25) (layer "F.Cu") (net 3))
 (segment (start 47.01 38.705) (end 42.2 38.705) (width 0.25) (layer "F.Cu") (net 3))
 (segment (start 47.62 38.095) (end 47.01 38.705) (width 0.25) (layer "F.Cu") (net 3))
 (via (at 39.3 33.405) (size 0.8) (drill 0.4) (layers "F.Cu" "B.Cu") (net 3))
 (segment (start 47.62 38.095) (end 45.65 36.125) (width 0.25) (layer "B.Cu") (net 3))
 (segment (start 44.65 33.405) (end 39.3 33.405) (width 0.25) (layer "B.Cu") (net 3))
 (segment (start 45.65 34.405) (end 44.65 33.405) (width 0.25) (layer "B.Cu") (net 3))
 (segment (start 45.65 36.125) (end 45.65 34.405) (width 0.25) (layer "B.Cu") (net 3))
 (segment (start 41.25 37.265) (end 41.25 36.105) (width 0.25) (layer "F.Cu") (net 4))
 (segment (start 41.25 38.555) (end 41.25 37.265) (width 0.25) (layer "F.Cu") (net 4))
 (segment (start 46.19 39.205) (end 41.9 39.205) (width 0.25) (layer "F.Cu") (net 4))
 (segment (start 47.62 40.635) (end 46.19 39.205) (width 0.25) (layer "F.Cu") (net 4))
 (segment (start 38.75 38.655) (end 38.2 39.205) (width 0.25) (layer "F.Cu") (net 4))
 (segment (start 38.75 36.105) (end 38.8 36.055) (width 0.25) (layer "F.Cu") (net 4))
 (segment (start 38.75 37.265) (end 38.75 38.655) (width 0.25) (layer "F.Cu") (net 4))
 (segment (start 41.25 36.105) (end 41.2 36.055) (width 0.25) (layer "F.Cu") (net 4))
 (segment (start 38.75 37.265) (end 38.75 36.105) (width 0.25) (layer "F.Cu") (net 4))
 (segment (start 38.2 39.205) (end 38.2 39.805) (width 0.25) (layer "F.Cu") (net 4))
 (segment (start 41.9 39.205) (end 41.25 38.555) (width 0.25) (layer "F.Cu") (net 4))
 (via (at 38.2 39.805) (size 0.8) (drill 0.4) (layers "F.Cu" "B.Cu") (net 4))
 (segment (start 39.3 40.205) (end 38.6 40.205) (width 0.25) (layer "B.Cu") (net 4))
 (segment (start 38.6 40.205) (end 38.2 39.805) (width 0.25) (layer "B.Cu") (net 4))
 (segment (start 41.2 36.055) (end 41.2 38.305) (width 0.25) (layer "B.Cu") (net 4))
 (segment (start 41.2 38.305) (end 39.3 40.205) (width 0.25) (layer "B.Cu") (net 4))
 (segment (start 40.75 37.265) (end 40.75 39.305) (width 0.25) (layer "F.Cu") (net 5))
 (segment (start 42.175 40.055) (end 41.5 40.055) (width 0.25) (layer "F.Cu") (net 5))
 (segment (start 40.75 39.305) (end 41.5 40.055) (width 0.25) (layer "F.Cu") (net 5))
 (segment (start 41.5 40.055) (end 41 39.555) (width 0.25) (layer "F.Cu") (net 5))
 (segment (start 40.249999 39.555001) (end 40.25 37.265) (width 0.25) (layer "F.Cu") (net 6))
 (segment (start 33.35 41.605) (end 38.95 41.605) (width 0.25) (layer "F.Cu") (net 6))
 (segment (start 32.38 40.635) (end 33.35 41.605) (width 0.25) (layer "F.Cu") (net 6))
 (segment (start 40.249999 40.305001) (end 40.249999 39.555001) (width 0.25) (layer "F.Cu") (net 6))
 (segment (start 38.95 41.605) (end 40.249999 40.305001) (width 0.25) (layer "F.Cu") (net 6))
 (segment (start 34.1 37.505) (end 33.4 36.805) (width 0.25) (layer "B.Cu") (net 6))
 (segment (start 39.6 36.055) (end 39.6 36.905) (width 0.25) (layer "B.Cu") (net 6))
 (segment (start 39 37.505) (end 34.1 37.505) (width 0.25) (layer "B.Cu") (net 6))
 (segment (start 31.5 36.805) (end 31 37.305) (width 0.25) (layer "B.Cu") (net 6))
 (segment (start 31 37.305) (end 31 39.255) (width 0.25) (layer "B.Cu") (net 6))
 (segment (start 31 39.255) (end 32.38 40.635) (width 0.25) (layer "B.Cu") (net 6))
 (segment (start 39.6 36.905) (end 39 37.505) (width 0.25) (layer "B.Cu") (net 6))
 (segment (start 33.4 36.805) (end 31.5 36.805) (width 0.25) (layer "B.Cu") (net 6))
 (segment (start 35.19 40.905) (end 32.38 38.095) (width 0.25) (layer "F.Cu") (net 7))
 (segment (start 39.75 37.265) (end 39.75 39.655) (width 0.25) (layer "F.Cu") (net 7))
 (segment (start 38.5 40.905) (end 35.19 40.905) (width 0.25) (layer "F.Cu") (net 7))
 (segment (start 39.75 39.655) (end 38.5 40.905) (width 0.25) (layer "F.Cu") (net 7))
 (segment (start 32.38 38.095) (end 39.71 38.095) (width 0.25) (layer "B.Cu") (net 7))
 (segment (start 39.71 38.095) (end 40.4 37.405) (width 0.25) (layer "B.Cu") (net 7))
 (segment (start 40.4 37.405) (end 40.4 36.055) (width 0.25) (layer "B.Cu") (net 7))
 (segment (start 41.6 31.405) (end 41.3 31.105) (width 0.25) (layer "F.Cu") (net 9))
 (segment (start 41.3 31.105) (end 38.2 31.105) (width 0.25) (layer "F.Cu") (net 9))
 (segment (start 37.6 39.105) (end 38.25 38.455) (width 0.25) (layer "F.Cu") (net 9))
 (segment (start 34 37.605) (end 35.5 39.105) (width 0.25) (layer "F.Cu") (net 9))
 (segment (start 34 35.955) (end 34 37.605) (width 0.25) (layer "F.Cu") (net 9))
 (segment (start 32.38 35.555) (end 33.6 35.555) (width 0.25) (layer "F.Cu") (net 9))
 (segment (start 38.25 38.455) (end 38.25 37.265) (width 0.25) (layer "F.Cu") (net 9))
 (segment (start 35.5 39.105) (end 37.6 39.105) (width 0.25) (layer "F.Cu") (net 9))
 (segment (start 33.6 35.555) (end 34 35.955) (width 0.25) (layer "F.Cu") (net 9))
 (segment (start 35.2 34.105) (end 34.9 34.105) (width 0.25) (layer "F.Cu") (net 9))
 (segment (start 41.6 35.355) (end 41.6 31.405) (width 0.25) (layer "F.Cu") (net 9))
 (segment (start 38.2 31.105) (end 35.2 34.105) (width 0.25) (layer "F.Cu") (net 9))
 (via (at 34.9 34.105) (size 0.8) (drill 0.4) (layers "F.Cu" "B.Cu") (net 9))
 (segment (start 32.38 35.555) (end 33.83 34.105) (width 0.25) (layer "B.Cu") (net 9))
 (segment (start 33.83 34.105) (end 34.9 34.105) (width 0.25) (layer "B.Cu") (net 9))
 (segment (start 38 30.505) (end 41.6 30.505) (width 0.25) (layer "F.Cu") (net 10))
 (segment (start 37.75 38.055) (end 37.75 37.265) (width 0.25) (layer "F.Cu") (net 10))
 (segment (start 35.8 38.605) (end 37.2 38.605) (width 0.25) (layer "F.Cu") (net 10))
 (segment (start 37.2 38.605) (end 37.75 38.055) (width 0.25) (layer "F.Cu") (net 10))
 (segment (start 34.5 37.305) (end 35.8 38.605) (width 0.25) (layer "F.Cu") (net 10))
 (segment (start 32.38 33.015) (end 34.5 35.135) (width 0.25) (layer "F.Cu") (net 10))
 (segment (start 32.38 33.015) (end 35.49 33.015) (width 0.25) (layer "F.Cu") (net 10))
 (segment (start 34.5 35.135) (end 34.5 37.305) (width 0.25) (layer "F.Cu") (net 10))
 (segment (start 42.4 31.305) (end 42.4 35.355) (width 0.25) (layer "F.Cu") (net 10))
 (segment (start 41.6 30.505) (end 42.4 31.305) (width 0.25) (layer "F.Cu") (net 10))
 (segment (start 35.49 33.015) (end 38 30.505) (width 0.25) (layer "F.Cu") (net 10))
 (segment (start 43.825 41.555) (end 44.85 41.555) (width 0.25) (layer "F.Cu") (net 11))
 (segment (start 44.85 41.555) (end 45.3 41.105) (width 0.25) (layer "F.Cu") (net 11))
 (via (at 45.3 41.105) (size 0.8) (drill 0.4) (layers "F.Cu" "B.Cu") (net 11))
 (segment (start 39.7 34.205) (end 44.7 34.205) (width 0.25) (layer "B.Cu") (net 11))
 (segment (start 39.2 34.705) (end 39.7 34.205) (width 0.25) (layer "B.Cu") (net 11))
 (segment (start 45.3 41.105) (end 45.3 36.905) (width 0.25) (layer "B.Cu") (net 11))
 (segment (start 45.1 34.605) (end 45.1 36.705) (width 0.25) (layer "B.Cu") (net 11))
 (segment (start 45.3 36.905) (end 45.1 36.705) (width 0.25) (layer "B.Cu") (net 11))
 (segment (start 39.2 35.355) (end 39.2 34.705) (width 0.25) (layer "B.Cu") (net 11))
 (segment (start 44.7 34.205) (end 45.1 34.605) (width 0.25) (layer "B.Cu") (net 11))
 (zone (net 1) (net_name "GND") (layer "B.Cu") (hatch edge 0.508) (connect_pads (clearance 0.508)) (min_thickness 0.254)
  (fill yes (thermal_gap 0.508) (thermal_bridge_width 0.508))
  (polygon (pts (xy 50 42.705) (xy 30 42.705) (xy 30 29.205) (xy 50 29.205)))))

